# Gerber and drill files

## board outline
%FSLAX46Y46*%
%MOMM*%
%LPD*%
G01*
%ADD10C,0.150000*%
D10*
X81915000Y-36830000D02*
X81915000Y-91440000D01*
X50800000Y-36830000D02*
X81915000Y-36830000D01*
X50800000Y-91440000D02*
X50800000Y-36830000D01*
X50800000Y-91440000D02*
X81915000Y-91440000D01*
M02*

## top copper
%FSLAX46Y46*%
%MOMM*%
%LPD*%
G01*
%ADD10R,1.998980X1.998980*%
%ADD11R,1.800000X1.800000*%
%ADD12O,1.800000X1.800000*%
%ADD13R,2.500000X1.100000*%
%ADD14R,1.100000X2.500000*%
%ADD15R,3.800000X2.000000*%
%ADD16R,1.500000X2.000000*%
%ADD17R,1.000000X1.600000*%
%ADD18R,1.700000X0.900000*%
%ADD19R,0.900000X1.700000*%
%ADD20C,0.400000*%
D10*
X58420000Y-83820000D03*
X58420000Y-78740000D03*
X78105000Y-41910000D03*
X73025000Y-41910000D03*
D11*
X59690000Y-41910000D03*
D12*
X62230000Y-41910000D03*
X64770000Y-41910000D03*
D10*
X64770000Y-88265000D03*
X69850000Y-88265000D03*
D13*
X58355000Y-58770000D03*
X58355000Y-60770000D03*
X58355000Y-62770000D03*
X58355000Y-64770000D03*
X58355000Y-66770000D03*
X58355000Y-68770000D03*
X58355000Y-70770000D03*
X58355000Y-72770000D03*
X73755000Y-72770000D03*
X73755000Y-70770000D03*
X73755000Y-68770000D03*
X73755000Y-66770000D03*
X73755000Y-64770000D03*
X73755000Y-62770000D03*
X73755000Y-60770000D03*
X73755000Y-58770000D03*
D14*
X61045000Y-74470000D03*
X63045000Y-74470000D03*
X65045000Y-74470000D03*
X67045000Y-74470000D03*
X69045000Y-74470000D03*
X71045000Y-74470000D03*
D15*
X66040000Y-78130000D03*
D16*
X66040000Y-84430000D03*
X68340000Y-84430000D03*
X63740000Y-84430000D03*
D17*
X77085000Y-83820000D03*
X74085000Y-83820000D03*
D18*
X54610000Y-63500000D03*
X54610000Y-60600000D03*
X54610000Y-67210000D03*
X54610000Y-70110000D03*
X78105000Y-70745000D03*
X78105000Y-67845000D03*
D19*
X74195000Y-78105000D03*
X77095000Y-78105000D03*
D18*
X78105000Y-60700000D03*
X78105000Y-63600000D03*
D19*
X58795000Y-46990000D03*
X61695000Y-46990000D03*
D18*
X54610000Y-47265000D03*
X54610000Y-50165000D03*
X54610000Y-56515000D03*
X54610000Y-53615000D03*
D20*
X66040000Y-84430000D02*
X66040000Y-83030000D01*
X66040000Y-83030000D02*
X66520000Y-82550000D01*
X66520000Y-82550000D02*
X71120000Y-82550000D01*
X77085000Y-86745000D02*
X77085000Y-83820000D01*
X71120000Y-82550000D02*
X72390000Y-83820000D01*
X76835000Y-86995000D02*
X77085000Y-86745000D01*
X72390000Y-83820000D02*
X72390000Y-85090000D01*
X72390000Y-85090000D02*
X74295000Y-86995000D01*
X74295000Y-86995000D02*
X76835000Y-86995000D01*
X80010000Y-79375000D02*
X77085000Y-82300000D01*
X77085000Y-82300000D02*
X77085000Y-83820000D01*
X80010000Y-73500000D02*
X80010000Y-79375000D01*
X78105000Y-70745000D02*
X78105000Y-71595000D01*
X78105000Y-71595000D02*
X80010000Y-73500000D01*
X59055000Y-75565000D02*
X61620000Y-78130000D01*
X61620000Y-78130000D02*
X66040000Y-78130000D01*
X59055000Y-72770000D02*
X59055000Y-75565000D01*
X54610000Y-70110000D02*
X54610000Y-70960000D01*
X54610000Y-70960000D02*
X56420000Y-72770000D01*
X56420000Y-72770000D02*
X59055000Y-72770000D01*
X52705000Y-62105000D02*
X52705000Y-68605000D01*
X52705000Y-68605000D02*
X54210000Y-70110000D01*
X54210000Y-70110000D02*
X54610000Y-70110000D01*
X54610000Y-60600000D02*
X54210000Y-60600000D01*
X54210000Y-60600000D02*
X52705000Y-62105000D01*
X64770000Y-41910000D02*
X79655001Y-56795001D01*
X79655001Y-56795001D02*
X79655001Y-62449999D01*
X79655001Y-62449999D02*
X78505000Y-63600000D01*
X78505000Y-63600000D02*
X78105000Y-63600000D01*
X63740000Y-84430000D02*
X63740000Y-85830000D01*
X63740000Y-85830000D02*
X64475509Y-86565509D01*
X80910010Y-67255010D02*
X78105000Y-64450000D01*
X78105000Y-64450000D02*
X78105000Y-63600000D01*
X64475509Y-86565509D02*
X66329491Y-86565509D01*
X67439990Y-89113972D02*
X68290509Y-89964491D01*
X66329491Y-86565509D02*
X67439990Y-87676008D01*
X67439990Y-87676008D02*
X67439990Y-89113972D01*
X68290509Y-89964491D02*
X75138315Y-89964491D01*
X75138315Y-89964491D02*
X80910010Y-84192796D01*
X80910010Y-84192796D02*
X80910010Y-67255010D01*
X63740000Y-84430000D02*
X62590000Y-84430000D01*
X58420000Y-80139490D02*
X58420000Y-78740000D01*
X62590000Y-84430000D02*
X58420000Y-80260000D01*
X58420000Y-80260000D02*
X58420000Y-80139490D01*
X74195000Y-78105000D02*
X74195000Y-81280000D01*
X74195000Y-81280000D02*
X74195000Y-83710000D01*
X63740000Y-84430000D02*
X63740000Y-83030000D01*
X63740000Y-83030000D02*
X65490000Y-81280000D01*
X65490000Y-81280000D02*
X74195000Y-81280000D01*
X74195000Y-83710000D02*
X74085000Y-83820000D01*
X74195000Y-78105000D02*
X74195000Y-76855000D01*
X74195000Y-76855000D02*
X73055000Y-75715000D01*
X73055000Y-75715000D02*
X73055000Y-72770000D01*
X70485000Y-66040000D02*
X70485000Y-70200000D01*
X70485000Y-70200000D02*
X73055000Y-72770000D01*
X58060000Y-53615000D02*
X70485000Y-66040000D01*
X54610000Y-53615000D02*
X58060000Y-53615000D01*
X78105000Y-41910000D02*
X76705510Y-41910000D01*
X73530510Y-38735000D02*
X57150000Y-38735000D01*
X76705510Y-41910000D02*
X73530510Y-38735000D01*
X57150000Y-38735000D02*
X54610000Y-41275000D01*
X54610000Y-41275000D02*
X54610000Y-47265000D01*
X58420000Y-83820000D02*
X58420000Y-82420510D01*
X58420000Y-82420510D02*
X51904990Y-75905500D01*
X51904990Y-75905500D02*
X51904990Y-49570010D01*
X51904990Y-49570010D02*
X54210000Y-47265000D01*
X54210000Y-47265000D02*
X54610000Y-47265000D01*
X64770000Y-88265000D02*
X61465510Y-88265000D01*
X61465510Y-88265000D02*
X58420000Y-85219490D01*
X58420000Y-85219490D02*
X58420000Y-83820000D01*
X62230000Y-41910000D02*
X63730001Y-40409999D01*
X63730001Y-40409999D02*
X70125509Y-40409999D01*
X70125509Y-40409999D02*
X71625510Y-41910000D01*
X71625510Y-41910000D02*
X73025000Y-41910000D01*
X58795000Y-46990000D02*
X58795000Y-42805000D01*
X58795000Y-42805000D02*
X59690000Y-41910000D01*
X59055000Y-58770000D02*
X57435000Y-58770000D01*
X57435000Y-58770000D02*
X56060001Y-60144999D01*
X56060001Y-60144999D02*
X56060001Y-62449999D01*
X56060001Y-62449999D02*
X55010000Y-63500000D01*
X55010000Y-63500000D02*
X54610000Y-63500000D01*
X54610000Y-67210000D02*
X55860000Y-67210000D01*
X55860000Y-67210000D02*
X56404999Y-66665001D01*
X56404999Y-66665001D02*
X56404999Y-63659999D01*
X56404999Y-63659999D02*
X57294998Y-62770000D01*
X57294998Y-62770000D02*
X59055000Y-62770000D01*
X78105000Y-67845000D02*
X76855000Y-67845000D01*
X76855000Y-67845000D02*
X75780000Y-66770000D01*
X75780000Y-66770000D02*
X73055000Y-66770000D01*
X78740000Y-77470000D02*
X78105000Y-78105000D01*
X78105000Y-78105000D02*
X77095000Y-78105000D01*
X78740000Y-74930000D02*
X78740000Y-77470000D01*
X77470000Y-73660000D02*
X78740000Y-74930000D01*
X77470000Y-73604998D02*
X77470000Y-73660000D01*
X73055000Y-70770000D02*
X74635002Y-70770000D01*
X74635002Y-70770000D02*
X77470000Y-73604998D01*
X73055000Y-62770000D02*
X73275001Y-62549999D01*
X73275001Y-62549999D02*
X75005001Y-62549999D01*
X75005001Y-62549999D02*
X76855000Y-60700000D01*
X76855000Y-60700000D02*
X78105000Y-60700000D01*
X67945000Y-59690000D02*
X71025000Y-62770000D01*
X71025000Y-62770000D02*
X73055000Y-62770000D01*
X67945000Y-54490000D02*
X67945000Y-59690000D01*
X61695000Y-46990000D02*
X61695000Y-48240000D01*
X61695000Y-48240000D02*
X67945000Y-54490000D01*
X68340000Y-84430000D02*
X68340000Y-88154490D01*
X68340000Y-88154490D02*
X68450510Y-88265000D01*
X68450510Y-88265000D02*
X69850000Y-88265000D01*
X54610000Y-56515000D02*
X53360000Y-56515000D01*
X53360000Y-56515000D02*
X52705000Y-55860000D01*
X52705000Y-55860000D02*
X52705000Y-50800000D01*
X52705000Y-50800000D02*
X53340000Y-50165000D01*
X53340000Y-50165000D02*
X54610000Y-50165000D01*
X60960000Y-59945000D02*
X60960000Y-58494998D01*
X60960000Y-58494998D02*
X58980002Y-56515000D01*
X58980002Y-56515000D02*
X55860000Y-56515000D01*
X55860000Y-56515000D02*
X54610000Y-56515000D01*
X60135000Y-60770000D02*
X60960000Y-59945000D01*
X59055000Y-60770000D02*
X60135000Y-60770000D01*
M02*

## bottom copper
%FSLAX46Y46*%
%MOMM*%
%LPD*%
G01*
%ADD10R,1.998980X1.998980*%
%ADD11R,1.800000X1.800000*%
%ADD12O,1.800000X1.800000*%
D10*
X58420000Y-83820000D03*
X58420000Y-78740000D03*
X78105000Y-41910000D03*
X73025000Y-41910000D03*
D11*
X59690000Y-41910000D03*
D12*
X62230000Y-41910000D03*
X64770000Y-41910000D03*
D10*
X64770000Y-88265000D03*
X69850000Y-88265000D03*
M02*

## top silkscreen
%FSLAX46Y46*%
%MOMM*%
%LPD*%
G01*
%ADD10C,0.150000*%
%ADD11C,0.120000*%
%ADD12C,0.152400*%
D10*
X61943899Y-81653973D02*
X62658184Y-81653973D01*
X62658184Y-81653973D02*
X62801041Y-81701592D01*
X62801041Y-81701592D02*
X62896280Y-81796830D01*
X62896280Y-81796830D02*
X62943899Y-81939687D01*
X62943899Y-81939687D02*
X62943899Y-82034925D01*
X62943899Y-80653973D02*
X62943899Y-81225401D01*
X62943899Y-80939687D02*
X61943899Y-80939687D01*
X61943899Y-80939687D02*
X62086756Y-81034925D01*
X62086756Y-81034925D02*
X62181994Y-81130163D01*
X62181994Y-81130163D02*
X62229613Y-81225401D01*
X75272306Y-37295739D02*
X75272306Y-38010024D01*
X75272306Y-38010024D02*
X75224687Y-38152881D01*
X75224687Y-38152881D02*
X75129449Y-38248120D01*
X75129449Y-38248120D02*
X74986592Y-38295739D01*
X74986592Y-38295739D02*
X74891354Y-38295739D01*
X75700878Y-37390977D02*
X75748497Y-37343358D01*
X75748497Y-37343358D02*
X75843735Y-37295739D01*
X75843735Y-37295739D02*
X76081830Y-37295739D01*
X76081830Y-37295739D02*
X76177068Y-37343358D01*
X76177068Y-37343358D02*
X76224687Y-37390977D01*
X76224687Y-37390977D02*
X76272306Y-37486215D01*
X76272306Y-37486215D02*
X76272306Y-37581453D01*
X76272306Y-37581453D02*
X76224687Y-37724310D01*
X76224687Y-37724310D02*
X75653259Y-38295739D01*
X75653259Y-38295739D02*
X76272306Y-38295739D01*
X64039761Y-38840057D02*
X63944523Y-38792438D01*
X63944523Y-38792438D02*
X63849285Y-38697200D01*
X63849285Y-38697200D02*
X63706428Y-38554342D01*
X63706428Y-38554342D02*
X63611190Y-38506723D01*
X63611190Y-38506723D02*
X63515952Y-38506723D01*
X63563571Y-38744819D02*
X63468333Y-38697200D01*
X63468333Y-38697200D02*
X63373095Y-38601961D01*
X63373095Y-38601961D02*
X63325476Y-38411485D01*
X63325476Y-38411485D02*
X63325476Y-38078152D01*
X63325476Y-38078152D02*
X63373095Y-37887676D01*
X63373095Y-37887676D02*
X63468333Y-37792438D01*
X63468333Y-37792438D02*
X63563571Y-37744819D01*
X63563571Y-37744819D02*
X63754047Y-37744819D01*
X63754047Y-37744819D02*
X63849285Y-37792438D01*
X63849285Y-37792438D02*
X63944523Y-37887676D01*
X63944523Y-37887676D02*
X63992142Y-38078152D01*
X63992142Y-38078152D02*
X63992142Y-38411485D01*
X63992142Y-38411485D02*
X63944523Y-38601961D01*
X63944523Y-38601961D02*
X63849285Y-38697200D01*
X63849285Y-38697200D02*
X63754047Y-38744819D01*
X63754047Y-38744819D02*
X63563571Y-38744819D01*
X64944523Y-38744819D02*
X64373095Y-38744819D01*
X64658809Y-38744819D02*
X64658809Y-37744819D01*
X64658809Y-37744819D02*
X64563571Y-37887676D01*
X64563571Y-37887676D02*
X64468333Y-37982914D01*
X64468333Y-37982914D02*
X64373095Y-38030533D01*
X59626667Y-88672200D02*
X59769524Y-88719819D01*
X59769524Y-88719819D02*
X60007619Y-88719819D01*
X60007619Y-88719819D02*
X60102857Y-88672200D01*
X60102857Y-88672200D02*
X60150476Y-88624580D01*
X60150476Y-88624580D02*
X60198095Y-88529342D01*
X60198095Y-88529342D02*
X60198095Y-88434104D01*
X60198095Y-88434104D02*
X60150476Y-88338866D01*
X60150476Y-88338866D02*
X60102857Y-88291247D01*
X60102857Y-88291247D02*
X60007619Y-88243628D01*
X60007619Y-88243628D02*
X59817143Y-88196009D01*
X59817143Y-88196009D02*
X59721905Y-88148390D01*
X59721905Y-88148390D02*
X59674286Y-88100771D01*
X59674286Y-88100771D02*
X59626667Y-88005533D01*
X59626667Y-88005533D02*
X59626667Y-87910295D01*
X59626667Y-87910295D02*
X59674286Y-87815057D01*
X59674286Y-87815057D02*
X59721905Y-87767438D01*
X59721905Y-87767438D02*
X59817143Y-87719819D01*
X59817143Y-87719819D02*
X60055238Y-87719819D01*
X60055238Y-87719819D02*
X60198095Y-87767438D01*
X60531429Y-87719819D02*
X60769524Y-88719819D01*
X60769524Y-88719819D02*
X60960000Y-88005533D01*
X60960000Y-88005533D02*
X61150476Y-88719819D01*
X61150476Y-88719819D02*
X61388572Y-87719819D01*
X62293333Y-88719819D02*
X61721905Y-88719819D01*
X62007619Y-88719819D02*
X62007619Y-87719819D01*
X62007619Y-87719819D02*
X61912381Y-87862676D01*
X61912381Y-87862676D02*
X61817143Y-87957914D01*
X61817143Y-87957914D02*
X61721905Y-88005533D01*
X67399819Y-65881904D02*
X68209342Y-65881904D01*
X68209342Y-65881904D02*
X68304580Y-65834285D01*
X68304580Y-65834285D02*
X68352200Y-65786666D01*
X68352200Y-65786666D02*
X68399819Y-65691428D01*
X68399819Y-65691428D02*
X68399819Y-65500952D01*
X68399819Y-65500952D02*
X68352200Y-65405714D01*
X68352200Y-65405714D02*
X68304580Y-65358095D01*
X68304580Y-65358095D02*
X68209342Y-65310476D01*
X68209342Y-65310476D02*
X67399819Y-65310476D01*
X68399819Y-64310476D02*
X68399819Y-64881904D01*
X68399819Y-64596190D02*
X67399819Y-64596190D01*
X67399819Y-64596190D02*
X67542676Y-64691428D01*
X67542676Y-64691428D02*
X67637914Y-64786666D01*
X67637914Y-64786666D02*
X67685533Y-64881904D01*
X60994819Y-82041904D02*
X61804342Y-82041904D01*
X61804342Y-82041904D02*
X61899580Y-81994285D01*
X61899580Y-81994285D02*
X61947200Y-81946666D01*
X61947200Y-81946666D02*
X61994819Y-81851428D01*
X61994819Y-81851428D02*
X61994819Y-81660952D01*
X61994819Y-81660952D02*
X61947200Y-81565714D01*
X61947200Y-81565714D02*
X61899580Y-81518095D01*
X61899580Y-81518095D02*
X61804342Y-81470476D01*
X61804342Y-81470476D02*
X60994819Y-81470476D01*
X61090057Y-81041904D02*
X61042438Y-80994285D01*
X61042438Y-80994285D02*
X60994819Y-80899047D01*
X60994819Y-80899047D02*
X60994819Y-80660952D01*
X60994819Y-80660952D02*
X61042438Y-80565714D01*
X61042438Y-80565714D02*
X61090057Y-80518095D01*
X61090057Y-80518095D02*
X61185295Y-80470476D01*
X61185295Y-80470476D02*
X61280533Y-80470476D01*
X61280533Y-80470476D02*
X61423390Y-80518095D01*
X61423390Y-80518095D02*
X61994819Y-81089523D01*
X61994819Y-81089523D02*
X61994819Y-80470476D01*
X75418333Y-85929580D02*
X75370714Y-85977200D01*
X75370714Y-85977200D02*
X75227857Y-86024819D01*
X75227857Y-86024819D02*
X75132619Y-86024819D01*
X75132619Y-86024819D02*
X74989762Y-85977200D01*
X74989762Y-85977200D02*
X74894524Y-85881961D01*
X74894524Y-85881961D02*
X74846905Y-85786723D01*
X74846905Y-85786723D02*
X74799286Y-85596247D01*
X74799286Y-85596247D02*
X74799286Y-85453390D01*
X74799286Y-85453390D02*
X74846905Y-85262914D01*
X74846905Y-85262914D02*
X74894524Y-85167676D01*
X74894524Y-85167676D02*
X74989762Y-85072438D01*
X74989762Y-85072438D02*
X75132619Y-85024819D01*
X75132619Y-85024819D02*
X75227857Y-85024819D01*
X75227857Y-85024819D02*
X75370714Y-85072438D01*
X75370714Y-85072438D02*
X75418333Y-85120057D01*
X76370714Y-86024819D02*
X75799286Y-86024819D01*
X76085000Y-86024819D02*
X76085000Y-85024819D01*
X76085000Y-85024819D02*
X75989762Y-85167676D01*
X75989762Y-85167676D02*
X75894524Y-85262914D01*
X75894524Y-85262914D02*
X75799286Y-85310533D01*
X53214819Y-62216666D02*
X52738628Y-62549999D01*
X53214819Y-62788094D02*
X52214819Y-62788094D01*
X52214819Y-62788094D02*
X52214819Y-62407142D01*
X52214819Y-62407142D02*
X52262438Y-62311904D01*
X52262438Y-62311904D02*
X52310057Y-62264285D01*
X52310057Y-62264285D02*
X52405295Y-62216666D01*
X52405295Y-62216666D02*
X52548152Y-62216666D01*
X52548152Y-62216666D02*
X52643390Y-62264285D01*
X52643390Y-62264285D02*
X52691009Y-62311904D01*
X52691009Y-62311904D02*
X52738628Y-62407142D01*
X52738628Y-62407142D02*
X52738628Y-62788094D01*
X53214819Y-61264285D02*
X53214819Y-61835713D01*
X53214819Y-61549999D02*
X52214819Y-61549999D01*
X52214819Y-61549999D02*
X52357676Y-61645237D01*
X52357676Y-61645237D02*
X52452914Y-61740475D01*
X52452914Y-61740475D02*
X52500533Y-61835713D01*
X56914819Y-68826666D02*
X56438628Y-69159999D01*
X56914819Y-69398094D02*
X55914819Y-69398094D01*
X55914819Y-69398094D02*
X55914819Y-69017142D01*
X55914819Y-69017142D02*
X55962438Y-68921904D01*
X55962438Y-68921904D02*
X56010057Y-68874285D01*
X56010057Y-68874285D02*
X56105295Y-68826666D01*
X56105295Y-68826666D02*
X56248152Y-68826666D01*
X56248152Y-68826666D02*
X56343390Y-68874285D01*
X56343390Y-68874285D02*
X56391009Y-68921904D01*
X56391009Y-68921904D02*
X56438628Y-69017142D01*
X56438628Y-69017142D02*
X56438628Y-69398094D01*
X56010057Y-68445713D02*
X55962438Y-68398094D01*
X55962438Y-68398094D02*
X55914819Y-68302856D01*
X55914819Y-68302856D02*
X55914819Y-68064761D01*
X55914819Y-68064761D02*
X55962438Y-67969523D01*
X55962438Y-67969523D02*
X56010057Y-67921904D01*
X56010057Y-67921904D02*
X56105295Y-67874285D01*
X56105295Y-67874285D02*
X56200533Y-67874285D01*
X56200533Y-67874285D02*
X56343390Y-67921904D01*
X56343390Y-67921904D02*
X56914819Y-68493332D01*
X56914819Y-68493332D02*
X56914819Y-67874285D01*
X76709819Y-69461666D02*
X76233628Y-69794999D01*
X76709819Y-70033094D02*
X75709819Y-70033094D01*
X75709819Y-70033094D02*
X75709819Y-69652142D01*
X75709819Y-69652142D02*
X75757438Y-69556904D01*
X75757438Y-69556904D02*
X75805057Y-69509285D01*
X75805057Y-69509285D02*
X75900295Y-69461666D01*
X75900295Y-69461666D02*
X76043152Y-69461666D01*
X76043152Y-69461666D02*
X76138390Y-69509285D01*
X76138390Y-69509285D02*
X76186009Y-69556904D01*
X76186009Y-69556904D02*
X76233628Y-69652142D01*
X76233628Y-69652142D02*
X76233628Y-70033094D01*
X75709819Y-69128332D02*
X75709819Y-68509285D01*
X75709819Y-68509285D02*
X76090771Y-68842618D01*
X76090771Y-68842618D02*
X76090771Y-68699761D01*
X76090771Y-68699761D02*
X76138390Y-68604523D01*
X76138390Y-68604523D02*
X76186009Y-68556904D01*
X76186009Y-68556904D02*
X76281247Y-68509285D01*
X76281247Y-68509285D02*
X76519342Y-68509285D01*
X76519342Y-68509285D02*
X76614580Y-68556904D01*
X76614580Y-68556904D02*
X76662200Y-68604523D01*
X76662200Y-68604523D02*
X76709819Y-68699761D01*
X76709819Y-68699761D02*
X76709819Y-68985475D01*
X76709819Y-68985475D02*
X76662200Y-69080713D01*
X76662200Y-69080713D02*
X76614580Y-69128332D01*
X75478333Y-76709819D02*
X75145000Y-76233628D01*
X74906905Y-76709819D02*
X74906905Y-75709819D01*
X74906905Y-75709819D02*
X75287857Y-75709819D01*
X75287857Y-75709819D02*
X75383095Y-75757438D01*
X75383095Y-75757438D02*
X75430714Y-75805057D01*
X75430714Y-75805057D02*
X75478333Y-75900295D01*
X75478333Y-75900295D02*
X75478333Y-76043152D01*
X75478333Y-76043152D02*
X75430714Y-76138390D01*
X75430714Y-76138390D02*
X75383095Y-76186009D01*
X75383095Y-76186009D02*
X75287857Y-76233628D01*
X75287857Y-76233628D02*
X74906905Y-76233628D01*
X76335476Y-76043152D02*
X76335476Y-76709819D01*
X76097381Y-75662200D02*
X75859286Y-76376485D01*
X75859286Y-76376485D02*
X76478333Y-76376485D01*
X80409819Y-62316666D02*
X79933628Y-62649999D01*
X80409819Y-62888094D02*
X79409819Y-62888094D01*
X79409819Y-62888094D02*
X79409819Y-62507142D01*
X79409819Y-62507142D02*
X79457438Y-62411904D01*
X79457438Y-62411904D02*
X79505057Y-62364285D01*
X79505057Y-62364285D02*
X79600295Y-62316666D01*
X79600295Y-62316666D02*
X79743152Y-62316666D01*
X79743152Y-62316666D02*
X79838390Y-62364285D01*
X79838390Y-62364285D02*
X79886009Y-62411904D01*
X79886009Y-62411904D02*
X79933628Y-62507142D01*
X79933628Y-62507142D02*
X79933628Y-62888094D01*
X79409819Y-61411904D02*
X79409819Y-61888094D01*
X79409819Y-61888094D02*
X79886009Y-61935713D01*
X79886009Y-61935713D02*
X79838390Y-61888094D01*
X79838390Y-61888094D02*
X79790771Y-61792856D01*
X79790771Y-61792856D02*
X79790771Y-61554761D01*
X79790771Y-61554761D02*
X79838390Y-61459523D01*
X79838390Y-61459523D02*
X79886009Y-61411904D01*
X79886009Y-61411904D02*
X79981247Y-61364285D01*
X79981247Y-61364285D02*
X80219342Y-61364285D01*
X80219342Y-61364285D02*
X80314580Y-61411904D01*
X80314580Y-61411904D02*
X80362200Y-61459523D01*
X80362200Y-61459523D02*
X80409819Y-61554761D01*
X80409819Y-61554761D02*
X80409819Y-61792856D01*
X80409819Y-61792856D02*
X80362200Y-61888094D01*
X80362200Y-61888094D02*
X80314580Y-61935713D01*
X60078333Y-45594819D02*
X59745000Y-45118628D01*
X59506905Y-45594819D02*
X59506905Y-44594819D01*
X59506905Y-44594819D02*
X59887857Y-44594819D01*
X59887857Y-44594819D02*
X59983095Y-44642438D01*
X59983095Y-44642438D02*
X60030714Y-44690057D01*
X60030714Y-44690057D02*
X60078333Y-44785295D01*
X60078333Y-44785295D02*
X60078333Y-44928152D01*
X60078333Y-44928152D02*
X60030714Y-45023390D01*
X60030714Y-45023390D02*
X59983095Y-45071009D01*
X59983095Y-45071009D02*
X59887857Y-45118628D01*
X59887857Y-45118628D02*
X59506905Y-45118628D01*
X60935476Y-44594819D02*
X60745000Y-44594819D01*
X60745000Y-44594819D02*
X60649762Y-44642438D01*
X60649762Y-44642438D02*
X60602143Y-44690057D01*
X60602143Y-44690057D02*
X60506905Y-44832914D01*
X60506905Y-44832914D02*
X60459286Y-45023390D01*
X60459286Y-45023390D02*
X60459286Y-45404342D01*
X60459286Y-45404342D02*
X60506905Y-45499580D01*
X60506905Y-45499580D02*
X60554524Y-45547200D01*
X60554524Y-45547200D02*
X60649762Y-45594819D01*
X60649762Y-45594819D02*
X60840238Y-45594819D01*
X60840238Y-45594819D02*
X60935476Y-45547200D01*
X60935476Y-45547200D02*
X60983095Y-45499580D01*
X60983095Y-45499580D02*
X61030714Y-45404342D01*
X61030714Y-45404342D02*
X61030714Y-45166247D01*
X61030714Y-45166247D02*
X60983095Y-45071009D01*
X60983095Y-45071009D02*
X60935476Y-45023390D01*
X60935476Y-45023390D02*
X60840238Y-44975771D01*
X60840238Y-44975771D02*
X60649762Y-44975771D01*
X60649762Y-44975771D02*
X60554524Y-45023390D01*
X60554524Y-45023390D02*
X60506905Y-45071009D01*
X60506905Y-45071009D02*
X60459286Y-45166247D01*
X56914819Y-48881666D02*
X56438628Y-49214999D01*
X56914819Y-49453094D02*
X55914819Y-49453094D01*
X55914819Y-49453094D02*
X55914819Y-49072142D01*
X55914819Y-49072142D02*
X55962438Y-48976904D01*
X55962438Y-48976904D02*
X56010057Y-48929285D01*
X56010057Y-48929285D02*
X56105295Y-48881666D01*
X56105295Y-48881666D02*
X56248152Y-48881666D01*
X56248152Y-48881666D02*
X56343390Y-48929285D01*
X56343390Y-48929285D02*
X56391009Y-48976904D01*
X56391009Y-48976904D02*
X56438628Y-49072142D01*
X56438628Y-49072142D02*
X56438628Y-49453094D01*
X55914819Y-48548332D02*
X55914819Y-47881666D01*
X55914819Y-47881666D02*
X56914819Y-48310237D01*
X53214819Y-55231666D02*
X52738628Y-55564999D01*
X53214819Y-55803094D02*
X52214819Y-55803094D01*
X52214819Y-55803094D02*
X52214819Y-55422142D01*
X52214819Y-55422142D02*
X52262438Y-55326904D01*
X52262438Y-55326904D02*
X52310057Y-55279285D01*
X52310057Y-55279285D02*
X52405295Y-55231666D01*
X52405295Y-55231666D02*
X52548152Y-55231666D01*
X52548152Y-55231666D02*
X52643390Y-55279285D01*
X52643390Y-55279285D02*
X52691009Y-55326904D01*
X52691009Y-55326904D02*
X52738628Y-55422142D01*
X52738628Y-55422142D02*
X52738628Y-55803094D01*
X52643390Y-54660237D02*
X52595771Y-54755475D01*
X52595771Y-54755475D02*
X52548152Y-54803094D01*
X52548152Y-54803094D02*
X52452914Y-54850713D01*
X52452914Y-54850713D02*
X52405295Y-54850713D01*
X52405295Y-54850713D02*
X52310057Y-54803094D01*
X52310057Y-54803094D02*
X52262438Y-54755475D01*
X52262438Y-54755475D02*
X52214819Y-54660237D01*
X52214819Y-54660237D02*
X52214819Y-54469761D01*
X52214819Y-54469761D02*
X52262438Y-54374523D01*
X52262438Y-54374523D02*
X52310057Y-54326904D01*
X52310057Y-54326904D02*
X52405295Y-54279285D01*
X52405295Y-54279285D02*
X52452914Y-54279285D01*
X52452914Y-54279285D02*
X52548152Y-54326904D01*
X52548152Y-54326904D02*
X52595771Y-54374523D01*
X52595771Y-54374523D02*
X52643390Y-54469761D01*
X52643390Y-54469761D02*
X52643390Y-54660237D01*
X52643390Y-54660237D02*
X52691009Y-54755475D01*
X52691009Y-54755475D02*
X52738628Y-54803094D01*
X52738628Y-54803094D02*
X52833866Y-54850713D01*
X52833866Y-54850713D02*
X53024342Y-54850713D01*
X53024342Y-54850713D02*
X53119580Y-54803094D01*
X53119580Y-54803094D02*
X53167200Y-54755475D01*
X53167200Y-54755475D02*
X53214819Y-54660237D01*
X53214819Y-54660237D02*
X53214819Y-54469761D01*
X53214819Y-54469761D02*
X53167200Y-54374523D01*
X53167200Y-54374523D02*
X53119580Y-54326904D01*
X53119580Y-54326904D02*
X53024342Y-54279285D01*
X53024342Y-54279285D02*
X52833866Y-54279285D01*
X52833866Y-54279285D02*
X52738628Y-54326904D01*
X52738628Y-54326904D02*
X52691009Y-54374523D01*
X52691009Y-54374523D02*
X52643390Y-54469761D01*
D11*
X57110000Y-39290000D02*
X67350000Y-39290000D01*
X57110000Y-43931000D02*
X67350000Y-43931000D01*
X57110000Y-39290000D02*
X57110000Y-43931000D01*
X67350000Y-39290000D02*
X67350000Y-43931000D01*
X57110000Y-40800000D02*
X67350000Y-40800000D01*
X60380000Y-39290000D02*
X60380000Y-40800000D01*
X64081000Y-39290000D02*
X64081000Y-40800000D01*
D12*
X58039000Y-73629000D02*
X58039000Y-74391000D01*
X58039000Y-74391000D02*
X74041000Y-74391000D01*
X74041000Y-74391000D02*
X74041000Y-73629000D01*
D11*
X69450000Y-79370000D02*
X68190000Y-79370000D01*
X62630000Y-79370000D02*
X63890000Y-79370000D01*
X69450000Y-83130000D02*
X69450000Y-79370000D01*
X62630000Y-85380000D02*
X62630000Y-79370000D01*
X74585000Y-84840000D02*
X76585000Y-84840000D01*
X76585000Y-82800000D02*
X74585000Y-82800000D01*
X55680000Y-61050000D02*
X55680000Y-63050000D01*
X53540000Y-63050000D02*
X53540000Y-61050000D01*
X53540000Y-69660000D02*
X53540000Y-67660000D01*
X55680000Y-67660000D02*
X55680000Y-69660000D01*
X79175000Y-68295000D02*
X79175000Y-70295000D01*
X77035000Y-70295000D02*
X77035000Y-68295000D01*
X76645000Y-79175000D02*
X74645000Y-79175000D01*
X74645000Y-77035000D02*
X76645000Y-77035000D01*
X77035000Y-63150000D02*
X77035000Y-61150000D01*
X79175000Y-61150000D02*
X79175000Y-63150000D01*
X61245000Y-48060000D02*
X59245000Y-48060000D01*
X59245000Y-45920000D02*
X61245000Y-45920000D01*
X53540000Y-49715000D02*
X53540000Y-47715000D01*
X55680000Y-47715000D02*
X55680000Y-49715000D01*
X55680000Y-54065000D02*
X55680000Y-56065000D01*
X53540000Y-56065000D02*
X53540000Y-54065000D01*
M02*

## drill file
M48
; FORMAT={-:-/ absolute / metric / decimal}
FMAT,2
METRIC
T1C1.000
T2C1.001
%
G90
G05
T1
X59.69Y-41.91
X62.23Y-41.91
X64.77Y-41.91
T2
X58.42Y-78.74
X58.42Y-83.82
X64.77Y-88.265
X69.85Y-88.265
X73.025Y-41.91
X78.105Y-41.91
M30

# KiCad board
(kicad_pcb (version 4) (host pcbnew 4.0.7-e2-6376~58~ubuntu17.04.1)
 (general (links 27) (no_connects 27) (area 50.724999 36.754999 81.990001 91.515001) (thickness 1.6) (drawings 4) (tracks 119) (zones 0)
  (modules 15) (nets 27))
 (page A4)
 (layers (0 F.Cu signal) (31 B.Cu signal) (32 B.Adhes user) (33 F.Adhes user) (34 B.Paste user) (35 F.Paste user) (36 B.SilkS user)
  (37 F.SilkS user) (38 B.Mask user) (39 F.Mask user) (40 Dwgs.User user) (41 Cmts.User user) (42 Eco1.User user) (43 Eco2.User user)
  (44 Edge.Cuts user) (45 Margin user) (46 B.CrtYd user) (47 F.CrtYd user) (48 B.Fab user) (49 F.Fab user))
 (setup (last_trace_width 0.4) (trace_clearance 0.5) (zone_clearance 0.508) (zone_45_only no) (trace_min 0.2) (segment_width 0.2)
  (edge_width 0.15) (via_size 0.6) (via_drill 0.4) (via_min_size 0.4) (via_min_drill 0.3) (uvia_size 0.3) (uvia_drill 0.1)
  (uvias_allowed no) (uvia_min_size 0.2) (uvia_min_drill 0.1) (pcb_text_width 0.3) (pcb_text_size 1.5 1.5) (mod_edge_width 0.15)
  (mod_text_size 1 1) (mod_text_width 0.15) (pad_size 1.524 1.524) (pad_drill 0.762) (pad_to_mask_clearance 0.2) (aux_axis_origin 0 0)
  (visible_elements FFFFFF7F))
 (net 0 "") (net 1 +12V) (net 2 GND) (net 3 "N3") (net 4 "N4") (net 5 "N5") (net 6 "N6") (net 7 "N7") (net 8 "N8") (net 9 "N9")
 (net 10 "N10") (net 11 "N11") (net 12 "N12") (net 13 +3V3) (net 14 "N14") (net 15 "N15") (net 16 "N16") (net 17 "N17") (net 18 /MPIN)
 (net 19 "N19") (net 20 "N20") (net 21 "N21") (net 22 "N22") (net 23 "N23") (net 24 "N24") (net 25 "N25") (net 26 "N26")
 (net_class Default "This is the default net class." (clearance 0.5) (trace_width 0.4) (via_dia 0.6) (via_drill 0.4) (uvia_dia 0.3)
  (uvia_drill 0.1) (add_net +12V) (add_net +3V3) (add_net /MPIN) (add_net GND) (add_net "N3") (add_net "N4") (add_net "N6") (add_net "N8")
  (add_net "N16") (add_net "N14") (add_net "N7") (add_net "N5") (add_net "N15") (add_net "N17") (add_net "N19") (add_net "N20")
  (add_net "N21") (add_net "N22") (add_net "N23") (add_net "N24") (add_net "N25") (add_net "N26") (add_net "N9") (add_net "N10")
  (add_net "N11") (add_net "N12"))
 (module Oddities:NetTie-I (layer F.Cu) (at 58.42 81.28 90)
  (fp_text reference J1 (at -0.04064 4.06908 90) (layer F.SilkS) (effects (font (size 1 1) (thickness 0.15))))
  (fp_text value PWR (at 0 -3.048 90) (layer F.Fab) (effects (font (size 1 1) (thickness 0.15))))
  (pad 1 thru_hole rect (at -2.54 0 90) (size 1.99898 1.99898) (drill 1.00076) (layers *.Cu *.Mask) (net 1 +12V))
  (pad 2 thru_hole rect (at 2.54 0 90) (size 1.99898 1.99898) (drill 1.00076) (layers *.Cu *.Mask) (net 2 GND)))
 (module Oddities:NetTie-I (layer F.Cu) (at 75.565 41.91 180)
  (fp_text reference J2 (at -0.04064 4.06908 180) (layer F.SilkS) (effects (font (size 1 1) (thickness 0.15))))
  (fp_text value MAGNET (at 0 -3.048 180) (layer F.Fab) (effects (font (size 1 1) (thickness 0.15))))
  (pad 1 thru_hole rect (at -2.54 0 180) (size 1.99898 1.99898) (drill 1.00076) (layers *.Cu *.Mask) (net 1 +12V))
  (pad 2 thru_hole rect (at 2.54 0 180) (size 1.99898 1.99898) (drill 1.00076) (layers *.Cu *.Mask) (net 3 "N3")))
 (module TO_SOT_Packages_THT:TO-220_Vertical (layer F.Cu) (at 59.69 41.91)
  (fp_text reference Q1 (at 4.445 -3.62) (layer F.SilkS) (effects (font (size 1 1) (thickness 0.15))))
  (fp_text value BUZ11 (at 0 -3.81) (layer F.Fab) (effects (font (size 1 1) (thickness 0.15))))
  (fp_line (start -2.58 -2.62) (end 7.66 -2.62) (layer F.SilkS) (width 0.12))
  (fp_line (start -2.58 2.021) (end 7.66 2.021) (layer F.SilkS) (width 0.12))
  (fp_line (start -2.58 -2.62) (end -2.58 2.021) (layer F.SilkS) (width 0.12))
  (fp_line (start 7.66 -2.62) (end 7.66 2.021) (layer F.SilkS) (width 0.12))
  (fp_line (start -2.58 -1.11) (end 7.66 -1.11) (layer F.SilkS) (width 0.12))
  (fp_line (start 0.69 -2.62) (end 0.69 -1.11) (layer F.SilkS) (width 0.12))
  (fp_line (start 4.391 -2.62) (end 4.391 -1.11) (layer F.SilkS) (width 0.12))
  (pad 1 thru_hole rect (at 0 0) (size 1.8 1.8) (drill 1) (layers *.Cu *.Mask) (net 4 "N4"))
  (pad 2 thru_hole oval (at 2.54 0) (size 1.8 1.8) (drill 1) (layers *.Cu *.Mask) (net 3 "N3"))
  (pad 3 thru_hole oval (at 5.08 0) (size 1.8 1.8) (drill 1) (layers *.Cu *.Mask) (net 2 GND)))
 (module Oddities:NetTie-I (layer F.Cu) (at 67.31 88.265)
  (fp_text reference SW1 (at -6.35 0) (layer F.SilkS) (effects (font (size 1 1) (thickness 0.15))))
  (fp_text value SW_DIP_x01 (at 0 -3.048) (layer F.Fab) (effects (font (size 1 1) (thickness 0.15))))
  (pad 1 thru_hole rect (at -2.54 0) (size 1.99898 1.99898) (drill 1.00076) (layers *.Cu *.Mask) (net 1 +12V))
  (pad 2 thru_hole rect (at 2.54 0) (size 1.99898 1.99898) (drill 1.00076) (layers *.Cu *.Mask) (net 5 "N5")))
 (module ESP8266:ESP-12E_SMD (layer F.Cu) (at 59.055 58.77)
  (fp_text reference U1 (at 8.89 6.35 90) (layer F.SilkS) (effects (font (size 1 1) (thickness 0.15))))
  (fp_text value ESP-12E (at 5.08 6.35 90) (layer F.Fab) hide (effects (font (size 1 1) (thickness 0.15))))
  (fp_line (start -1.016 14.859) (end -1.016 15.621) (layer F.SilkS) (width 0.1524))
  (fp_line (start -1.016 15.621) (end 14.986 15.621) (layer F.SilkS) (width 0.1524))
  (fp_line (start 14.986 15.621) (end 14.986 14.859) (layer F.SilkS) (width 0.1524))
  (pad 1 smd rect (at 0 0) (size 2.5 1.1) (drill (offset -0.7 0)) (layers F.Cu F.Paste F.Mask) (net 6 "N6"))
  (pad 2 smd rect (at 0 2) (size 2.5 1.1) (drill (offset -0.7 0)) (layers F.Cu F.Paste F.Mask) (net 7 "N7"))
  (pad 3 smd rect (at 0 4) (size 2.5 1.1) (drill (offset -0.7 0)) (layers F.Cu F.Paste F.Mask) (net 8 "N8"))
  (pad 4 smd rect (at 0 6) (size 2.5 1.1) (drill (offset -0.7 0)) (layers F.Cu F.Paste F.Mask) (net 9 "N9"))
  (pad 5 smd rect (at 0 8) (size 2.5 1.1) (drill (offset -0.7 0)) (layers F.Cu F.Paste F.Mask) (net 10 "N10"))
  (pad 6 smd rect (at 0 10) (size 2.5 1.1) (drill (offset -0.7 0)) (layers F.Cu F.Paste F.Mask) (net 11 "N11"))
  (pad 7 smd rect (at 0 12) (size 2.5 1.1) (drill (offset -0.7 0)) (layers F.Cu F.Paste F.Mask) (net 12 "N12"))
  (pad 8 smd rect (at 0 14) (size 2.5 1.1) (drill (offset -0.7 0)) (layers F.Cu F.Paste F.Mask) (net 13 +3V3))
  (pad 9 smd rect (at 14 14) (size 2.5 1.1) (drill (offset 0.7 0)) (layers F.Cu F.Paste F.Mask) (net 2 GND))
  (pad 10 smd rect (at 14 12) (size 2.5 1.1) (drill (offset 0.7 0)) (layers F.Cu F.Paste F.Mask) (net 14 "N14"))
  (pad 11 smd rect (at 14 10) (size 2.5 1.1) (drill (offset 0.7 0)) (layers F.Cu F.Paste F.Mask) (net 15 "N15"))
  (pad 12 smd rect (at 14 8) (size 2.5 1.1) (drill (offset 0.7 0)) (layers F.Cu F.Paste F.Mask) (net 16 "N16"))
  (pad 13 smd rect (at 14 6) (size 2.5 1.1) (drill (offset 0.7 0)) (layers F.Cu F.Paste F.Mask) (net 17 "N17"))
  (pad 14 smd rect (at 14 4) (size 2.5 1.1) (drill (offset 0.7 0)) (layers F.Cu F.Paste F.Mask) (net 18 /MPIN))
  (pad 15 smd rect (at 14 2) (size 2.5 1.1) (drill (offset 0.7 0)) (layers F.Cu F.Paste F.Mask) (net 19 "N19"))
  (pad 16 smd rect (at 14 0) (size 2.5 1.1) (drill (offset 0.7 0)) (layers F.Cu F.Paste F.Mask) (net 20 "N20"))
  (pad 17 smd rect (at 1.99 15 90) (size 2.5 1.1) (drill (offset -0.7 0)) (layers F.Cu F.Paste F.Mask) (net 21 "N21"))
  (pad 18 smd rect (at 3.99 15 90) (size 2.5 1.1) (drill (offset -0.7 0)) (layers F.Cu F.Paste F.Mask) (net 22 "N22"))
  (pad 19 smd rect (at 5.99 15 90) (size 2.5 1.1) (drill (offset -0.7 0)) (layers F.Cu F.Paste F.Mask) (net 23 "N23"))
  (pad 20 smd rect (at 7.99 15 90) (size 2.5 1.1) (drill (offset -0.7 0)) (layers F.Cu F.Paste F.Mask) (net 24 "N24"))
  (pad 21 smd rect (at 9.99 15 90) (size 2.5 1.1) (drill (offset -0.7 0)) (layers F.Cu F.Paste F.Mask) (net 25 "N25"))
  (pad 22 smd rect (at 11.99 15 90) (size 2.5 1.1) (drill (offset -0.7 0)) (layers F.Cu F.Paste F.Mask) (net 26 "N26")))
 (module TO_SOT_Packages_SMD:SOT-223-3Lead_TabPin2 (layer F.Cu) (at 66.04 81.28 90)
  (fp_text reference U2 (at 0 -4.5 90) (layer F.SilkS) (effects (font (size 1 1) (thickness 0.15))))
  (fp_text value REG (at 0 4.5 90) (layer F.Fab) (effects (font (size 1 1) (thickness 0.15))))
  (fp_line (start 1.91 3.41) (end 1.91 2.15) (layer F.SilkS) (width 0.12))
  (fp_line (start 1.91 -3.41) (end 1.91 -2.15) (layer F.SilkS) (width 0.12))
  (fp_line (start -1.85 3.41) (end 1.91 3.41) (layer F.SilkS) (width 0.12))
  (fp_line (start -4.1 -3.41) (end 1.91 -3.41) (layer F.SilkS) (width 0.12))
  (pad 2 smd rect (at 3.15 0 90) (size 2 3.8) (layers F.Cu F.Paste F.Mask) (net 13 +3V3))
  (pad 2 smd rect (at -3.15 0 90) (size 2 1.5) (layers F.Cu F.Paste F.Mask) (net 13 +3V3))
  (pad 3 smd rect (at -3.15 2.3 90) (size 2 1.5) (layers F.Cu F.Paste F.Mask) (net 5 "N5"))
  (pad 1 smd rect (at -3.15 -2.3 90) (size 2 1.5) (layers F.Cu F.Paste F.Mask) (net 2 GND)))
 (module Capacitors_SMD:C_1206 (layer F.Cu) (at 75.585 83.82 180)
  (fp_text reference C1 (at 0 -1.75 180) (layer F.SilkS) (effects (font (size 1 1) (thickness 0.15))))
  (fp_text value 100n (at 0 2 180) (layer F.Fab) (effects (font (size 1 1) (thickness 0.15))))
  (fp_line (start 1 -1.02) (end -1 -1.02) (layer F.SilkS) (width 0.12))
  (fp_line (start -1 1.02) (end 1 1.02) (layer F.SilkS) (width 0.12))
  (pad 1 smd rect (at -1.5 0 180) (size 1 1.6) (layers F.Cu F.Paste F.Mask) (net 13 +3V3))
  (pad 2 smd rect (at 1.5 0 180) (size 1 1.6) (layers F.Cu F.Paste F.Mask) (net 2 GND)))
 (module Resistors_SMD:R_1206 (layer F.Cu) (at 54.61 62.05 90)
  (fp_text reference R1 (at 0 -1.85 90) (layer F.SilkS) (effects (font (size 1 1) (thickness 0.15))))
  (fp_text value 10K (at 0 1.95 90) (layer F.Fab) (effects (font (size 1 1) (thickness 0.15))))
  (fp_line (start 1 1.07) (end -1 1.07) (layer F.SilkS) (width 0.12))
  (fp_line (start -1 -1.07) (end 1 -1.07) (layer F.SilkS) (width 0.12))
  (pad 1 smd rect (at -1.45 0 90) (size 0.9 1.7) (layers F.Cu F.Paste F.Mask) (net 6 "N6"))
  (pad 2 smd rect (at 1.45 0 90) (size 0.9 1.7) (layers F.Cu F.Paste F.Mask) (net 13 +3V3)))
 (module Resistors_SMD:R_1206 (layer F.Cu) (at 54.61 68.66 270)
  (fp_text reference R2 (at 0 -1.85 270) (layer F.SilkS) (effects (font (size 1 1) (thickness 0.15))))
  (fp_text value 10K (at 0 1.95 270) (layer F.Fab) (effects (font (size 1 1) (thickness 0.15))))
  (fp_line (start 1 1.07) (end -1 1.07) (layer F.SilkS) (width 0.12))
  (fp_line (start -1 -1.07) (end 1 -1.07) (layer F.SilkS) (width 0.12))
  (pad 1 smd rect (at -1.45 0 270) (size 0.9 1.7) (layers F.Cu F.Paste F.Mask) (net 8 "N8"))
  (pad 2 smd rect (at 1.45 0 270) (size 0.9 1.7) (layers F.Cu F.Paste F.Mask) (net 13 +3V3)))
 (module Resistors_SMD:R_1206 (layer F.Cu) (at 78.105 69.295 90)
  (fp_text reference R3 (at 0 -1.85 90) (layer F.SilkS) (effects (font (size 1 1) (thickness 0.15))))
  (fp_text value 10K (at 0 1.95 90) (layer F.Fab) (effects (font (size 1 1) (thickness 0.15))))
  (fp_line (start 1 1.07) (end -1 1.07) (layer F.SilkS) (width 0.12))
  (fp_line (start -1 -1.07) (end 1 -1.07) (layer F.SilkS) (width 0.12))
  (pad 1 smd rect (at -1.45 0 90) (size 0.9 1.7) (layers F.Cu F.Paste F.Mask) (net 13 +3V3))
  (pad 2 smd rect (at 1.45 0 90) (size 0.9 1.7) (layers F.Cu F.Paste F.Mask) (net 16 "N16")))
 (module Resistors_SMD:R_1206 (layer F.Cu) (at 75.645 78.105)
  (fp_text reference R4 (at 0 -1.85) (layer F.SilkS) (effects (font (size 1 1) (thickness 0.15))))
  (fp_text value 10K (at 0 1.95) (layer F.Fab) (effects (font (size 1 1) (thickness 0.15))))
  (fp_line (start 1 1.07) (end -1 1.07) (layer F.SilkS) (width 0.12))
  (fp_line (start -1 -1.07) (end 1 -1.07) (layer F.SilkS) (width 0.12))
  (pad 1 smd rect (at -1.45 0) (size 0.9 1.7) (layers F.Cu F.Paste F.Mask) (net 2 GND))
  (pad 2 smd rect (at 1.45 0) (size 0.9 1.7) (layers F.Cu F.Paste F.Mask) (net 14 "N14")))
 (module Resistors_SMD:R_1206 (layer F.Cu) (at 78.105 62.15 270)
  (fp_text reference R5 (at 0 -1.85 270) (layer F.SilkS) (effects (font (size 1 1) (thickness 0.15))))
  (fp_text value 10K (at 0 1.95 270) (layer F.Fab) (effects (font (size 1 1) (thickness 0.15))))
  (fp_line (start 1 1.07) (end -1 1.07) (layer F.SilkS) (width 0.12))
  (fp_line (start -1 -1.07) (end 1 -1.07) (layer F.SilkS) (width 0.12))
  (pad 1 smd rect (at -1.45 0 270) (size 0.9 1.7) (layers F.Cu F.Paste F.Mask) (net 18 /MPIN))
  (pad 2 smd rect (at 1.45 0 270) (size 0.9 1.7) (layers F.Cu F.Paste F.Mask) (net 2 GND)))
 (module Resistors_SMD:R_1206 (layer F.Cu) (at 60.245 46.99)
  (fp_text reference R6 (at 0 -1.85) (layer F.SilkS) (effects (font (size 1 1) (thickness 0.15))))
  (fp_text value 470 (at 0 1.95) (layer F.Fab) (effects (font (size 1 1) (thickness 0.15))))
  (fp_line (start 1 1.07) (end -1 1.07) (layer F.SilkS) (width 0.12))
  (fp_line (start -1 -1.07) (end 1 -1.07) (layer F.SilkS) (width 0.12))
  (pad 1 smd rect (at -1.45 0) (size 0.9 1.7) (layers F.Cu F.Paste F.Mask) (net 4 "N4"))
  (pad 2 smd rect (at 1.45 0) (size 0.9 1.7) (layers F.Cu F.Paste F.Mask) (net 18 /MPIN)))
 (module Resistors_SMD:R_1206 (layer F.Cu) (at 54.61 48.715 270)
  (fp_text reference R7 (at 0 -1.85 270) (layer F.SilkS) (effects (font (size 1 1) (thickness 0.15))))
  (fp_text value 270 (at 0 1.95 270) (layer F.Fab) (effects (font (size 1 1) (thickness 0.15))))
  (fp_line (start 1 1.07) (end -1 1.07) (layer F.SilkS) (width 0.12))
  (fp_line (start -1 -1.07) (end 1 -1.07) (layer F.SilkS) (width 0.12))
  (pad 1 smd rect (at -1.45 0 270) (size 0.9 1.7) (layers F.Cu F.Paste F.Mask) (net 1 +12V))
  (pad 2 smd rect (at 1.45 0 270) (size 0.9 1.7) (layers F.Cu F.Paste F.Mask) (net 7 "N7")))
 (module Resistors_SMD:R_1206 (layer F.Cu) (at 54.61 55.065 90)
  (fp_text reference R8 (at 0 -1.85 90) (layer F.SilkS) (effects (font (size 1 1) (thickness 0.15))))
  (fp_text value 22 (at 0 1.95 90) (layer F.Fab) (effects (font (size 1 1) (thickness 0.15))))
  (fp_line (start 1 1.07) (end -1 1.07) (layer F.SilkS) (width 0.12))
  (fp_line (start -1 -1.07) (end 1 -1.07) (layer F.SilkS) (width 0.12))
  (pad 1 smd rect (at -1.45 0 90) (size 0.9 1.7) (layers F.Cu F.Paste F.Mask) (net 7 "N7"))
  (pad 2 smd rect (at 1.45 0 90) (size 0.9 1.7) (layers F.Cu F.Paste F.Mask) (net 2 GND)))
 (gr_line (start 81.915 36.83) (end 81.915 91.44) (layer Edge.Cuts) (width 0.15))
 (gr_line (start 50.8 36.83) (end 81.915 36.83) (layer Edge.Cuts) (width 0.15))
 (gr_line (start 50.8 91.44) (end 50.8 36.83) (layer Edge.Cuts) (width 0.15))
 (gr_line (start 50.8 91.44) (end 81.915 91.44) (layer Edge.Cuts) (width 0.15))
 (segment (start 66.04 84.43) (end 66.04 83.03) (width 0.4) (layer F.Cu) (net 13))
 (segment (start 66.04 83.03) (end 66.52 82.55) (width 0.4) (layer F.Cu) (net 13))
 (segment (start 66.52 82.55) (end 71.12 82.55) (width 0.4) (layer F.Cu) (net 13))
 (segment (start 77.085 86.745) (end 77.085 83.82) (width 0.4) (layer F.Cu) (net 13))
 (segment (start 71.12 82.55) (end 72.39 83.82) (width 0.4) (layer F.Cu) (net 13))
 (segment (start 76.835 86.995) (end 77.085 86.745) (width 0.4) (layer F.Cu) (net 13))
 (segment (start 72.39 83.82) (end 72.39 85.09) (width 0.4) (layer F.Cu) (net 13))
 (segment (start 72.39 85.09) (end 74.295 86.995) (width 0.4) (layer F.Cu) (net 13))
 (segment (start 74.295 86.995) (end 76.835 86.995) (width 0.4) (layer F.Cu) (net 13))
 (segment (start 80.01 79.375) (end 77.085 82.3) (width 0.4) (layer F.Cu) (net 13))
 (segment (start 77.085 82.3) (end 77.085 83.82) (width 0.4) (layer F.Cu) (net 13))
 (segment (start 80.01 73.5) (end 80.01 79.375) (width 0.4) (layer F.Cu) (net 13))
 (segment (start 78.105 70.745) (end 78.105 71.595) (width 0.4) (layer F.Cu) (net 13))
 (segment (start 78.105 71.595) (end 80.01 73.5) (width 0.4) (layer F.Cu) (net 13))
 (segment (start 59.055 75.565) (end 61.62 78.13) (width 0.4) (layer F.Cu) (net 13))
 (segment (start 61.62 78.13) (end 66.04 78.13) (width 0.4) (layer F.Cu) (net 13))
 (segment (start 59.055 72.77) (end 59.055 75.565) (width 0.4) (layer F.Cu) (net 13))
 (segment (start 54.61 70.11) (end 54.61 70.96) (width 0.4) (layer F.Cu) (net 13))
 (segment (start 54.61 70.96) (end 56.42 72.77) (width 0.4) (layer F.Cu) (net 13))
 (segment (start 56.42 72.77) (end 59.055 72.77) (width 0.4) (layer F.Cu) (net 13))
 (segment (start 52.705 62.105) (end 52.705 68.605) (width 0.4) (layer F.Cu) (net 13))
 (segment (start 52.705 68.605) (end 54.21 70.11) (width 0.4) (layer F.Cu) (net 13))
 (segment (start 54.21 70.11) (end 54.61 70.11) (width 0.4) (layer F.Cu) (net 13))
 (segment (start 54.61 60.6) (end 54.21 60.6) (width 0.4) (layer F.Cu) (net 13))
 (segment (start 54.21 60.6) (end 52.705 62.105) (width 0.4) (layer F.Cu) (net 13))
 (segment (start 64.77 41.91) (end 79.655001 56.795001) (width 0.4) (layer F.Cu) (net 2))
 (segment (start 79.655001 56.795001) (end 79.655001 62.449999) (width 0.4) (layer F.Cu) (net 2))
 (segment (start 79.655001 62.449999) (end 78.505 63.6) (width 0.4) (layer F.Cu) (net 2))
 (segment (start 78.505 63.6) (end 78.105 63.6) (width 0.4) (layer F.Cu) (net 2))
 (segment (start 63.74 84.43) (end 63.74 85.83) (width 0.4) (layer F.Cu) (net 2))
 (segment (start 63.74 85.83) (end 64.475509 86.565509) (width 0.4) (layer F.Cu) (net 2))
 (segment (start 80.91001 67.25501) (end 78.105 64.45) (width 0.4) (layer F.Cu) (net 2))
 (segment (start 78.105 64.45) (end 78.105 63.6) (width 0.4) (layer F.Cu) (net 2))
 (segment (start 64.475509 86.565509) (end 66.329491 86.565509) (width 0.4) (layer F.Cu) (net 2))
 (segment (start 67.43999 89.113972) (end 68.290509 89.964491) (width 0.4) (layer F.Cu) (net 2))
 (segment (start 66.329491 86.565509) (end 67.43999 87.676008) (width 0.4) (layer F.Cu) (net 2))
 (segment (start 67.43999 87.676008) (end 67.43999 89.113972) (width 0.4) (layer F.Cu) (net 2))
 (segment (start 68.290509 89.964491) (end 75.138315 89.964491) (width 0.4) (layer F.Cu) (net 2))
 (segment (start 75.138315 89.964491) (end 80.91001 84.192796) (width 0.4) (layer F.Cu) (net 2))
 (segment (start 80.91001 84.192796) (end 80.91001 67.25501) (width 0.4) (layer F.Cu) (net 2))
 (segment (start 63.74 84.43) (end 62.59 84.43) (width 0.4) (layer F.Cu) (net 2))
 (segment (start 58.42 80.13949) (end 58.42 78.74) (width 0.4) (layer F.Cu) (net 2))
 (segment (start 62.59 84.43) (end 58.42 80.26) (width 0.4) (layer F.Cu) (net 2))
 (segment (start 58.42 80.26) (end 58.42 80.13949) (width 0.4) (layer F.Cu) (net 2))
 (segment (start 74.195 78.105) (end 74.195 81.28) (width 0.4) (layer F.Cu) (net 2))
 (segment (start 74.195 81.28) (end 74.195 83.71) (width 0.4) (layer F.Cu) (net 2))
 (segment (start 63.74 84.43) (end 63.74 83.03) (width 0.4) (layer F.Cu) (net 2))
 (segment (start 63.74 83.03) (end 65.49 81.28) (width 0.4) (layer F.Cu) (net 2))
 (segment (start 65.49 81.28) (end 74.195 81.28) (width 0.4) (layer F.Cu) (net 2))
 (segment (start 74.195 83.71) (end 74.085 83.82) (width 0.4) (layer F.Cu) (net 2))
 (segment (start 74.195 78.105) (end 74.195 76.855) (width 0.4) (layer F.Cu) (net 2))
 (segment (start 74.195 76.855) (end 73.055 75.715) (width 0.4) (layer F.Cu) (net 2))
 (segment (start 73.055 75.715) (end 73.055 72.77) (width 0.4) (layer F.Cu) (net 2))
 (segment (start 70.485 66.04) (end 70.485 70.2) (width 0.4) (layer F.Cu) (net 2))
 (segment (start 70.485 70.2) (end 73.055 72.77) (width 0.4) (layer F.Cu) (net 2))
 (segment (start 58.06 53.615) (end 70.485 66.04) (width 0.4) (layer F.Cu) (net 2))
 (segment (start 54.61 53.615) (end 58.06 53.615) (width 0.4) (layer F.Cu) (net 2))
 (segment (start 78.105 41.91) (end 76.70551 41.91) (width 0.4) (layer F.Cu) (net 1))
 (segment (start 73.53051 38.735) (end 57.15 38.735) (width 0.4) (layer F.Cu) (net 1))
 (segment (start 76.70551 41.91) (end 73.53051 38.735) (width 0.4) (layer F.Cu) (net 1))
 (segment (start 57.15 38.735) (end 54.61 41.275) (width 0.4) (layer F.Cu) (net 1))
 (segment (start 54.61 41.275) (end 54.61 47.265) (width 0.4) (layer F.Cu) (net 1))
 (segment (start 58.42 83.82) (end 58.42 82.42051) (width 0.4) (layer F.Cu) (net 1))
 (segment (start 58.42 82.42051) (end 51.90499 75.9055) (width 0.4) (layer F.Cu) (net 1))
 (segment (start 51.90499 75.9055) (end 51.90499 49.57001) (width 0.4) (layer F.Cu) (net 1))
 (segment (start 51.90499 49.57001) (end 54.21 47.265) (width 0.4) (layer F.Cu) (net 1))
 (segment (start 54.21 47.265) (end 54.61 47.265) (width 0.4) (layer F.Cu) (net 1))
 (segment (start 64.77 88.265) (end 61.46551 88.265) (width 0.4) (layer F.Cu) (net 1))
 (segment (start 61.46551 88.265) (end 58.42 85.21949) (width 0.4) (layer F.Cu) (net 1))
 (segment (start 58.42 85.21949) (end 58.42 83.82) (width 0.4) (layer F.Cu) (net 1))
 (segment (start 62.23 41.91) (end 63.730001 40.409999) (width 0.4) (layer F.Cu) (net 3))
 (segment (start 63.730001 40.409999) (end 70.125509 40.409999) (width 0.4) (layer F.Cu) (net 3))
 (segment (start 70.125509 40.409999) (end 71.62551 41.91) (width 0.4) (layer F.Cu) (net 3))
 (segment (start 71.62551 41.91) (end 73.025 41.91) (width 0.4) (layer F.Cu) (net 3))
 (segment (start 58.795 46.99) (end 58.795 42.805) (width 0.4) (layer F.Cu) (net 4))
 (segment (start 58.795 42.805) (end 59.69 41.91) (width 0.4) (layer F.Cu) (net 4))
 (segment (start 59.055 58.77) (end 57.435 58.77) (width 0.4) (layer F.Cu) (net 6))
 (segment (start 57.435 58.77) (end 56.060001 60.144999) (width 0.4) (layer F.Cu) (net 6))
 (segment (start 56.060001 60.144999) (end 56.060001 62.449999) (width 0.4) (layer F.Cu) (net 6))
 (segment (start 56.060001 62.449999) (end 55.01 63.5) (width 0.4) (layer F.Cu) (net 6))
 (segment (start 55.01 63.5) (end 54.61 63.5) (width 0.4) (layer F.Cu) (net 6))
 (segment (start 54.61 67.21) (end 55.86 67.21) (width 0.4) (layer F.Cu) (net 8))
 (segment (start 55.86 67.21) (end 56.404999 66.665001) (width 0.4) (layer F.Cu) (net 8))
 (segment (start 56.404999 66.665001) (end 56.404999 63.659999) (width 0.4) (layer F.Cu) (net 8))
 (segment (start 56.404999 63.659999) (end 57.294998 62.77) (width 0.4) (layer F.Cu) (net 8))
 (segment (start 57.294998 62.77) (end 59.055 62.77) (width 0.4) (layer F.Cu) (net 8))
 (segment (start 78.105 67.845) (end 76.855 67.845) (width 0.4) (layer F.Cu) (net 16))
 (segment (start 76.855 67.845) (end 75.78 66.77) (width 0.4) (layer F.Cu) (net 16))
 (segment (start 75.78 66.77) (end 73.055 66.77) (width 0.4) (layer F.Cu) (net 16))
 (segment (start 78.74 77.47) (end 78.105 78.105) (width 0.4) (layer F.Cu) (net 14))
 (segment (start 78.105 78.105) (end 77.095 78.105) (width 0.4) (layer F.Cu) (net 14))
 (segment (start 78.74 74.93) (end 78.74 77.47) (width 0.4) (layer F.Cu) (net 14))
 (segment (start 77.47 73.66) (end 78.74 74.93) (width 0.4) (layer F.Cu) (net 14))
 (segment (start 77.47 73.604998) (end 77.47 73.66) (width 0.4) (layer F.Cu) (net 14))
 (segment (start 73.055 70.77) (end 74.635002 70.77) (width 0.4) (layer F.Cu) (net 14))
 (segment (start 74.635002 70.77) (end 77.47 73.604998) (width 0.4) (layer F.Cu) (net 14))
 (segment (start 73.055 62.77) (end 73.275001 62.549999) (width 0.4) (layer F.Cu) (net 18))
 (segment (start 73.275001 62.549999) (end 75.005001 62.549999) (width 0.4) (layer F.Cu) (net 18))
 (segment (start 75.005001 62.549999) (end 76.855 60.7) (width 0.4) (layer F.Cu) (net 18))
 (segment (start 76.855 60.7) (end 78.105 60.7) (width 0.4) (layer F.Cu) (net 18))
 (segment (start 67.945 59.69) (end 71.025 62.77) (width 0.4) (layer F.Cu) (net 18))
 (segment (start 71.025 62.77) (end 73.055 62.77) (width 0.4) (layer F.Cu) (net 18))
 (segment (start 67.945 54.49) (end 67.945 59.69) (width 0.4) (layer F.Cu) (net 18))
 (segment (start 61.695 46.99) (end 61.695 48.24) (width 0.4) (layer F.Cu) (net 18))
 (segment (start 61.695 48.24) (end 67.945 54.49) (width 0.4) (layer F.Cu) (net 18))
 (segment (start 68.34 84.43) (end 68.34 88.15449) (width 0.4) (layer F.Cu) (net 5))
 (segment (start 68.34 88.15449) (end 68.45051 88.265) (width 0.4) (layer F.Cu) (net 5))
 (segment (start 68.45051 88.265) (end 69.85 88.265) (width 0.4) (layer F.Cu) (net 5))
 (segment (start 54.61 56.515) (end 53.36 56.515) (width 0.4) (layer F.Cu) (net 7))
 (segment (start 53.36 56.515) (end 52.705 55.86) (width 0.4) (layer F.Cu) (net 7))
 (segment (start 52.705 55.86) (end 52.705 50.8) (width 0.4) (layer F.Cu) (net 7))
 (segment (start 52.705 50.8) (end 53.34 50.165) (width 0.4) (layer F.Cu) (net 7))
 (segment (start 53.34 50.165) (end 54.61 50.165) (width 0.4) (layer F.Cu) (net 7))
 (segment (start 60.96 59.945) (end 60.96 58.494998) (width 0.4) (layer F.Cu) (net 7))
 (segment (start 60.96 58.494998) (end 58.980002 56.515) (width 0.4) (layer F.Cu) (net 7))
 (segment (start 58.980002 56.515) (end 55.86 56.515) (width 0.4) (layer F.Cu) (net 7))
 (segment (start 55.86 56.515) (end 54.61 56.515) (width 0.4) (layer F.Cu) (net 7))
 (segment (start 60.135 60.77) (end 60.96 59.945) (width 0.4) (layer F.Cu) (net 7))
 (segment (start 59.055 60.77) (end 60.135 60.77) (width 0.4) (layer F.Cu) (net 7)))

